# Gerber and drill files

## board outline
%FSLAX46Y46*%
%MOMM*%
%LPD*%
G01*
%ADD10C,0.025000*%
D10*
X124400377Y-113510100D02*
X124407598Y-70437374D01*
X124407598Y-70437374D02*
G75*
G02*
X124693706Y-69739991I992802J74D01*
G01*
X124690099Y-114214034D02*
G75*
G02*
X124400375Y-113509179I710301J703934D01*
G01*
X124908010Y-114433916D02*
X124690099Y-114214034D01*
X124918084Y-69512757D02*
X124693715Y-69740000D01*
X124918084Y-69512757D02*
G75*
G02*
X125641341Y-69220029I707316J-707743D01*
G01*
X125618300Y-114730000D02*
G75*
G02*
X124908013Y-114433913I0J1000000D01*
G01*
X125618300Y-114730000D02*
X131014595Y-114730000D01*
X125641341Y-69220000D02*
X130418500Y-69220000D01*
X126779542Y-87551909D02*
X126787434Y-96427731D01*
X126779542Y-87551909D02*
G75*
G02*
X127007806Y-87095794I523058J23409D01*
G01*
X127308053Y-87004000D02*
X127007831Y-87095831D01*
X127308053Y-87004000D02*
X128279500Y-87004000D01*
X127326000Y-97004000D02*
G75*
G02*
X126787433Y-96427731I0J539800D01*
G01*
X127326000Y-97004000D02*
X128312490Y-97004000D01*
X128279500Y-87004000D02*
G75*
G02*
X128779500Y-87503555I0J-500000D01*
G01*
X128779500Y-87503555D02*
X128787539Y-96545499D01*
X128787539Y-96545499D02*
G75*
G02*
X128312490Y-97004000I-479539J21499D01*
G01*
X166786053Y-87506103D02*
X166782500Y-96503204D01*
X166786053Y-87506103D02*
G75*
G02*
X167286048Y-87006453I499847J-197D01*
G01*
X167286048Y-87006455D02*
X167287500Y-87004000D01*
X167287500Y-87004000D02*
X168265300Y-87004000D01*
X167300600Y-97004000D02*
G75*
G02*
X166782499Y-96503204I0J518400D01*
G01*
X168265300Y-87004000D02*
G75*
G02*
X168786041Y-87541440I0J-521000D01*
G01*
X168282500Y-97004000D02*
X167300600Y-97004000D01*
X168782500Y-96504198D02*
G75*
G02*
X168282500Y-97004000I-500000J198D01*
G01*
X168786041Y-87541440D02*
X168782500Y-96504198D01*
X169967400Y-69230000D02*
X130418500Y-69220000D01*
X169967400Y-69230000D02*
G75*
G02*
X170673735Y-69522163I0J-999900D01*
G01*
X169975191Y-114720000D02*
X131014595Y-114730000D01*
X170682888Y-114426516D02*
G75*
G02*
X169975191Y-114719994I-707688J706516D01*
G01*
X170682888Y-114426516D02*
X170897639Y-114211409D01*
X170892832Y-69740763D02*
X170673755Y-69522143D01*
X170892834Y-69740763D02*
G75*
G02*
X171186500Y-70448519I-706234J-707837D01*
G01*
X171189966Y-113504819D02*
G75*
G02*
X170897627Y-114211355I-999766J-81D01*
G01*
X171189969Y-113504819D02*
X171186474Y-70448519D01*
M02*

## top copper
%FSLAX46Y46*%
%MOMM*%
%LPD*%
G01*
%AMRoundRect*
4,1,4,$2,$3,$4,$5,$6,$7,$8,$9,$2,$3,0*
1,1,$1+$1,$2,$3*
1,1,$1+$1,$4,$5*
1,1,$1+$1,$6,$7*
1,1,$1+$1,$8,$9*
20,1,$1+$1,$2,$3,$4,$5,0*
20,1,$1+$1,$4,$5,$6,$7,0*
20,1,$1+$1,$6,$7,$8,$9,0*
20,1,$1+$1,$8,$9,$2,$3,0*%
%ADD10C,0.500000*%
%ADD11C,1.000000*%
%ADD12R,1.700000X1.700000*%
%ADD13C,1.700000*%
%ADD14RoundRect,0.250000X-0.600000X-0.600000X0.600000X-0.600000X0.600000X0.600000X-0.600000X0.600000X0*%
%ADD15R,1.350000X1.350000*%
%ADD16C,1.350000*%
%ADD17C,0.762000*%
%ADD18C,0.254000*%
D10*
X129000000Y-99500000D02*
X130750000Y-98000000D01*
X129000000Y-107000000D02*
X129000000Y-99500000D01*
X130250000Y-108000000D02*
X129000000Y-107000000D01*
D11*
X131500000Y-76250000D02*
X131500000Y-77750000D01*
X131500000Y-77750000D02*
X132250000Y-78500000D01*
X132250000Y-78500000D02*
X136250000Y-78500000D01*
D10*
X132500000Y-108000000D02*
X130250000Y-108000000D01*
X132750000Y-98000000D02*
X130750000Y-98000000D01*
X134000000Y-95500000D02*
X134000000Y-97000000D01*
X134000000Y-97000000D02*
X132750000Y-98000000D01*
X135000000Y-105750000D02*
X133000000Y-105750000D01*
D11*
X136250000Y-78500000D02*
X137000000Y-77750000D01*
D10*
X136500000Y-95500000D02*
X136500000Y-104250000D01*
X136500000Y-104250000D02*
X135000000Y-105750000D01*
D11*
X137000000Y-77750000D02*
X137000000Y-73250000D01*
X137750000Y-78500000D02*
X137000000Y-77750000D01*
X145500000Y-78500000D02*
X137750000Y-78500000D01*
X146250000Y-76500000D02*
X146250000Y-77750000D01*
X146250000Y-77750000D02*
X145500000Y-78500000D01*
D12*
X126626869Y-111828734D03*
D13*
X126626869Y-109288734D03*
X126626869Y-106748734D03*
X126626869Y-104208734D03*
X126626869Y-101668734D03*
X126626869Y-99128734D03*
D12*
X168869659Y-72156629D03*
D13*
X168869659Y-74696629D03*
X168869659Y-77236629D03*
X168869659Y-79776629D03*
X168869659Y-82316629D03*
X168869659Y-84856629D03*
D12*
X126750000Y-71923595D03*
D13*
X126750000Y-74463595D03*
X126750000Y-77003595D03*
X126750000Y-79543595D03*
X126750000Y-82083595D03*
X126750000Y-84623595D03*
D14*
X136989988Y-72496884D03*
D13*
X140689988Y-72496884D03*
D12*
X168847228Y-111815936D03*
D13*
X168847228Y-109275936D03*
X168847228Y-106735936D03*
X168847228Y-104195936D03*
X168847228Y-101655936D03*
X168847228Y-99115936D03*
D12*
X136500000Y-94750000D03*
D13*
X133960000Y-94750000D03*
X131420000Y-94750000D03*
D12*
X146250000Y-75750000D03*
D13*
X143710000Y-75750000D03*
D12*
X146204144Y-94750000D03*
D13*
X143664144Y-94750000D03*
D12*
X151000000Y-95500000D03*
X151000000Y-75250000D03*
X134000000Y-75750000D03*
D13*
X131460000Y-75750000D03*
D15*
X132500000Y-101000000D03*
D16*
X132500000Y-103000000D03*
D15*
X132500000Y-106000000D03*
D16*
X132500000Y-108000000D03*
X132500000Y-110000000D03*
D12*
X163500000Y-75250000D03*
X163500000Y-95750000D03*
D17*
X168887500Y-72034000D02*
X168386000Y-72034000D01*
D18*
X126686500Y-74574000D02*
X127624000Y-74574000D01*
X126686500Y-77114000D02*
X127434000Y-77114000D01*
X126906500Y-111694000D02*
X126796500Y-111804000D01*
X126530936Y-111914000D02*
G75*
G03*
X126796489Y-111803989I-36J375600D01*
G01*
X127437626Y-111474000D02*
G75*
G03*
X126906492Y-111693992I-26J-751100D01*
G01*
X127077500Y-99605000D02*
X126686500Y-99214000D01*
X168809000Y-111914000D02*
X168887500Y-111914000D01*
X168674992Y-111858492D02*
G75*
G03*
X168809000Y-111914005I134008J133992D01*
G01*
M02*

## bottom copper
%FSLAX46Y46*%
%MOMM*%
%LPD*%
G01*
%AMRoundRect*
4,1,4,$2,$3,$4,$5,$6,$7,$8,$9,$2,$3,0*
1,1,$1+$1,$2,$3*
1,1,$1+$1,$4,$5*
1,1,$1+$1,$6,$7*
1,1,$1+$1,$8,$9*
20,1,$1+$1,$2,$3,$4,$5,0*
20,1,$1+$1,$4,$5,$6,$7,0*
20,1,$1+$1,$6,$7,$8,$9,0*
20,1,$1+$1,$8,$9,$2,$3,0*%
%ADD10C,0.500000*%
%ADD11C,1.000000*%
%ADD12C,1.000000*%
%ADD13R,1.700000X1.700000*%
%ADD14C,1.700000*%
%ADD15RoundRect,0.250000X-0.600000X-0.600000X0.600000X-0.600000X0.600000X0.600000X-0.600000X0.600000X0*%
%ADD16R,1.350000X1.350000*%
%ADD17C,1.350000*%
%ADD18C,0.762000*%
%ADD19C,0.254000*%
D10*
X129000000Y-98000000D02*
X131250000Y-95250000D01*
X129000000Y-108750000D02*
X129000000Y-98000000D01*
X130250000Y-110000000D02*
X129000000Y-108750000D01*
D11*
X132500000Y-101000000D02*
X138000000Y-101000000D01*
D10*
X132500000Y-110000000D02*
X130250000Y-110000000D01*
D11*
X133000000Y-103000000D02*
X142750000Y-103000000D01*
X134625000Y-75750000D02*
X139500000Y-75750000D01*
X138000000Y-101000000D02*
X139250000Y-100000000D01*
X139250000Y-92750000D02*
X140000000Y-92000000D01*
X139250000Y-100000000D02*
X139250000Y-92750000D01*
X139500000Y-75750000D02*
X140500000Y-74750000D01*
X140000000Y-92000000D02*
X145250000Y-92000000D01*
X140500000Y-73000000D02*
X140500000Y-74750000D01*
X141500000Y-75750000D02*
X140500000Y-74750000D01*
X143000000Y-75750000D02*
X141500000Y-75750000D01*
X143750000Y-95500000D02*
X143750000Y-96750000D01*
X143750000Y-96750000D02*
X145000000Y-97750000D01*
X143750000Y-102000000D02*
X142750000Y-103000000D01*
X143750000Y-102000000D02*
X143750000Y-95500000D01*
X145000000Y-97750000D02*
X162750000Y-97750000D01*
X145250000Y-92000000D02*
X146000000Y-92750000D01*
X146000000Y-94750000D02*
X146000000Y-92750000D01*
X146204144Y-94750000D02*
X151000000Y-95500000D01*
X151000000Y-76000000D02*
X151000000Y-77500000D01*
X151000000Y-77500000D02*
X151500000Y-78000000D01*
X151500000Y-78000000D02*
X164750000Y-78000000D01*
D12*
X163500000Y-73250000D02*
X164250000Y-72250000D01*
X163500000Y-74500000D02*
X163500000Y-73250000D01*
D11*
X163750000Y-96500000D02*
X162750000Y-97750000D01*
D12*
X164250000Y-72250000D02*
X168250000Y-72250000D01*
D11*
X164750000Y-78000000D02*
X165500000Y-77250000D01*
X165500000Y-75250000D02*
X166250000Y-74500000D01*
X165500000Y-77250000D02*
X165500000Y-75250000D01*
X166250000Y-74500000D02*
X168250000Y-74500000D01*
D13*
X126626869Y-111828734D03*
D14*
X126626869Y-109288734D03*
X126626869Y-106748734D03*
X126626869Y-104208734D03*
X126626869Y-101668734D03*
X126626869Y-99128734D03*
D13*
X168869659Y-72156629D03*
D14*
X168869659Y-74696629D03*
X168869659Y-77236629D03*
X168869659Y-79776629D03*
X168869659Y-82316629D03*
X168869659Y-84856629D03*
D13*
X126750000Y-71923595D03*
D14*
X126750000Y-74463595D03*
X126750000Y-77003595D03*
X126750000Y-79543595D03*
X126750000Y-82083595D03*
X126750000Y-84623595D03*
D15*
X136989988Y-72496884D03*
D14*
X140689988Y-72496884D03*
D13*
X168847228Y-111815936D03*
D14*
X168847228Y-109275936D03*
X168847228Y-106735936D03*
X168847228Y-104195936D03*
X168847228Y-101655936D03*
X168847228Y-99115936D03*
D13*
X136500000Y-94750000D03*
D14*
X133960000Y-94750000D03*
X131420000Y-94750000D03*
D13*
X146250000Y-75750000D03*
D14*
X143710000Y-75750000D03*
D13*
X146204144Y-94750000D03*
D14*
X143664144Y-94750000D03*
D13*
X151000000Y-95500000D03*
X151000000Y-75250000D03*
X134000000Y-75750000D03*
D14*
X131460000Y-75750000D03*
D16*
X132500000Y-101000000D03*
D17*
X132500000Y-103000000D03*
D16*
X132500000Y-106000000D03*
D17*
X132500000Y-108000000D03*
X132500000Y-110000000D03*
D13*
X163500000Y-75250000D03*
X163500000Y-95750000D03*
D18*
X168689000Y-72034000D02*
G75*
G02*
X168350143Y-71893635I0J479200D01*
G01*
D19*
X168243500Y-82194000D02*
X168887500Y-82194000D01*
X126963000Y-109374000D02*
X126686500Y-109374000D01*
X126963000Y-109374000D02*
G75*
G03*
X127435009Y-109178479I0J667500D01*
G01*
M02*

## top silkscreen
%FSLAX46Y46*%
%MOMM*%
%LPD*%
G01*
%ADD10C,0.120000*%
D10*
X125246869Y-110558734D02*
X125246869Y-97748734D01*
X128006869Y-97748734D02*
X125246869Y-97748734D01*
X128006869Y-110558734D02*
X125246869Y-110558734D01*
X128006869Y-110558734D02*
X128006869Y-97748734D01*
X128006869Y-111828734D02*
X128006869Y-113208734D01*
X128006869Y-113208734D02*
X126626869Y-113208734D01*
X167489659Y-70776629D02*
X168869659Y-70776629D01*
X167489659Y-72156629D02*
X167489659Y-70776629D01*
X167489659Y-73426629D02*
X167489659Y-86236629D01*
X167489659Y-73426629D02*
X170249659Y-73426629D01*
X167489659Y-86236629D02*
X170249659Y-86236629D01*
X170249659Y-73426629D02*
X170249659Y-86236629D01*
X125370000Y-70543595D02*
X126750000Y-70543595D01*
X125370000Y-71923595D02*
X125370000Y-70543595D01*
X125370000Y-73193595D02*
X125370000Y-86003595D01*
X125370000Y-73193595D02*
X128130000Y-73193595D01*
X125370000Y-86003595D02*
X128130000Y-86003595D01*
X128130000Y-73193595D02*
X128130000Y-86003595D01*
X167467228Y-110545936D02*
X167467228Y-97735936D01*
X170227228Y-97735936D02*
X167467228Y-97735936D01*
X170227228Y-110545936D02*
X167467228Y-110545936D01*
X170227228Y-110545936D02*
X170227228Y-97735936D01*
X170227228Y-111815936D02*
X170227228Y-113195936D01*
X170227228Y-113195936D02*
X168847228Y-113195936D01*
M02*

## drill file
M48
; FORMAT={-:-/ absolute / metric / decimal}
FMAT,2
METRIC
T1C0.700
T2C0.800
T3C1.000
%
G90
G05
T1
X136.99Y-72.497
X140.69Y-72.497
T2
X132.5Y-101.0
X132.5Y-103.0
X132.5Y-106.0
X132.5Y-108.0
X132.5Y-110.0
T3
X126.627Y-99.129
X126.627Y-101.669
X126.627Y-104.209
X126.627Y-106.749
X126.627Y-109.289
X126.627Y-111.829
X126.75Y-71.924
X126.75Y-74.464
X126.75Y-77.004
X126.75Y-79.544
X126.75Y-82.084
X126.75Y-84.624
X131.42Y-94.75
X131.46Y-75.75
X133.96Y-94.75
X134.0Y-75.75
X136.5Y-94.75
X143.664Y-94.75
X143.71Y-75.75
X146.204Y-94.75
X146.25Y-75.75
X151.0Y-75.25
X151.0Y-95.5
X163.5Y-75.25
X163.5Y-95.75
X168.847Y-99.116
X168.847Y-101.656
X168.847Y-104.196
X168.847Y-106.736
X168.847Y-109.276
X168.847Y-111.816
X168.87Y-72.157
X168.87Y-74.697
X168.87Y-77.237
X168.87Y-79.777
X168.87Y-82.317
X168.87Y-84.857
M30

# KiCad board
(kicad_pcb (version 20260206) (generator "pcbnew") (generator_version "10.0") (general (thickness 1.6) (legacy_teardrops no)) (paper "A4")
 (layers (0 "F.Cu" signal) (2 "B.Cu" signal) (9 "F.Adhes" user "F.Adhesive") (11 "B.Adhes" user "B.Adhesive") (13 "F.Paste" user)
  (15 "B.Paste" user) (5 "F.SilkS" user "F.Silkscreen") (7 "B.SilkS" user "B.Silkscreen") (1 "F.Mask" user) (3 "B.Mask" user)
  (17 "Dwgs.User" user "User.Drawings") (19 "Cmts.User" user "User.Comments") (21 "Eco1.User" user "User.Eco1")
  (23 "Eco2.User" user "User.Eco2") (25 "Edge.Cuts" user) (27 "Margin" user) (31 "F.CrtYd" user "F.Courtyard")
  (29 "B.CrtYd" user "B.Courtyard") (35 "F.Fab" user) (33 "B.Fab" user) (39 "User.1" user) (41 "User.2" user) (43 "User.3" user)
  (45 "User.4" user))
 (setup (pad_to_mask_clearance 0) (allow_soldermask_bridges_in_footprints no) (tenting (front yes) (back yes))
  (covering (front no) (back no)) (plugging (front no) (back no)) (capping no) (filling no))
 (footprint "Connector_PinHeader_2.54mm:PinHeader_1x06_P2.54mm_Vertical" (layer "F.Cu") (at 126.626869 111.828734 180)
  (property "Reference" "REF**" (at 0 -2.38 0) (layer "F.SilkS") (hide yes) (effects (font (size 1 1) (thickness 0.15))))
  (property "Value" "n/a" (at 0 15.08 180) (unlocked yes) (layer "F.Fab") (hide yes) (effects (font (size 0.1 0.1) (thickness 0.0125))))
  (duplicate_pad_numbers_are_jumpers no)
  (fp_line (start 1.38 1.27) (end 1.38 14.08) (stroke (width 0.12) (type solid)) (layer "F.SilkS"))
  (fp_line (start -1.38 14.08) (end 1.38 14.08) (stroke (width 0.12) (type solid)) (layer "F.SilkS"))
  (fp_line (start -1.38 1.27) (end 1.38 1.27) (stroke (width 0.12) (type solid)) (layer "F.SilkS"))
  (fp_line (start -1.38 1.27) (end -1.38 14.08) (stroke (width 0.12) (type solid)) (layer "F.SilkS"))
  (fp_line (start -1.38 0) (end -1.38 -1.38) (stroke (width 0.12) (type solid)) (layer "F.SilkS"))
  (fp_line (start -1.38 -1.38) (end 0 -1.38) (stroke (width 0.12) (type solid)) (layer "F.SilkS"))
  (pad "1" thru_hole rect (at 0 0 180) (size 1.7 1.7) (drill 1) (layers "*.Cu" "*.Mask") (remove_unused_layers no))
  (pad "2" thru_hole circle (at 0 2.54 180) (size 1.7 1.7) (drill 1) (layers "*.Cu" "*.Mask") (remove_unused_layers no))
  (pad "3" thru_hole circle (at 0 5.08 180) (size 1.7 1.7) (drill 1) (layers "*.Cu" "*.Mask") (remove_unused_layers no))
  (pad "4" thru_hole circle (at 0 7.62 180) (size 1.7 1.7) (drill 1) (layers "*.Cu" "*.Mask") (remove_unused_layers no))
  (pad "5" thru_hole circle (at 0 10.16 180) (size 1.7 1.7) (drill 1) (layers "*.Cu" "*.Mask") (remove_unused_layers no))
  (pad "6" thru_hole circle (at 0 12.7 180) (size 1.7 1.7) (drill 1) (layers "*.Cu" "*.Mask") (remove_unused_layers no)))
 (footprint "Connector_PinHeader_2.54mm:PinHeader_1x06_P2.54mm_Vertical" (layer "F.Cu") (at 168.869659 72.156629)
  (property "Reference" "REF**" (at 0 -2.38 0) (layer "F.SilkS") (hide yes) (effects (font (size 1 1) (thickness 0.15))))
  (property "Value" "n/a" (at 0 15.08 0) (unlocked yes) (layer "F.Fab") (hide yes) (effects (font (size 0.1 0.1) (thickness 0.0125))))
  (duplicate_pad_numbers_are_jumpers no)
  (fp_line (start -1.38 -1.38) (end 0 -1.38) (stroke (width 0.12) (type solid)) (layer "F.SilkS"))
  (fp_line (start -1.38 0) (end -1.38 -1.38) (stroke (width 0.12) (type solid)) (layer "F.SilkS"))
  (fp_line (start -1.38 1.27) (end -1.38 14.08) (stroke (width 0.12) (type solid)) (layer "F.SilkS"))
  (fp_line (start -1.38 1.27) (end 1.38 1.27) (stroke (width 0.12) (type solid)) (layer "F.SilkS"))
  (fp_line (start -1.38 14.08) (end 1.38 14.08) (stroke (width 0.12) (type solid)) (layer "F.SilkS"))
  (fp_line (start 1.38 1.27) (end 1.38 14.08) (stroke (width 0.12) (type solid)) (layer "F.SilkS"))
  (pad "1" thru_hole rect (at 0 0) (size 1.7 1.7) (drill 1) (layers "*.Cu" "*.Mask") (remove_unused_layers no))
  (pad "2" thru_hole circle (at 0 2.54) (size 1.7 1.7) (drill 1) (layers "*.Cu" "*.Mask") (remove_unused_layers no))
  (pad "3" thru_hole circle (at 0 5.08) (size 1.7 1.7) (drill 1) (layers "*.Cu" "*.Mask") (remove_unused_layers no))
  (pad "4" thru_hole circle (at 0 7.62) (size 1.7 1.7) (drill 1) (layers "*.Cu" "*.Mask") (remove_unused_layers no))
  (pad "5" thru_hole circle (at 0 10.16) (size 1.7 1.7) (drill 1) (layers "*.Cu" "*.Mask") (remove_unused_layers no))
  (pad "6" thru_hole circle (at 0 12.7) (size 1.7 1.7) (drill 1) (layers "*.Cu" "*.Mask") (remove_unused_layers no)))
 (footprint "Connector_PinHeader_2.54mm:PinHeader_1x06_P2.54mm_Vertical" (layer "F.Cu") (at 126.75 71.923595)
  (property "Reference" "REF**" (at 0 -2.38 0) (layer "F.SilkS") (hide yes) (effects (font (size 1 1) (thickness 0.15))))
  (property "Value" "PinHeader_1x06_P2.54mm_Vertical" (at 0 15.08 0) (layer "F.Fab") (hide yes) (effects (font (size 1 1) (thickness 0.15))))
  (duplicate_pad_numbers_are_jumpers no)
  (fp_line (start -1.38 -1.38) (end 0 -1.38) (stroke (width 0.12) (type solid)) (layer "F.SilkS"))
  (fp_line (start -1.38 0) (end -1.38 -1.38) (stroke (width 0.12) (type solid)) (layer "F.SilkS"))
  (fp_line (start -1.38 1.27) (end -1.38 14.08) (stroke (width 0.12) (type solid)) (layer "F.SilkS"))
  (fp_line (start -1.38 1.27) (end 1.38 1.27) (stroke (width 0.12) (type solid)) (layer "F.SilkS"))
  (fp_line (start -1.38 14.08) (end 1.38 14.08) (stroke (width 0.12) (type solid)) (layer "F.SilkS"))
  (fp_line (start 1.38 1.27) (end 1.38 14.08) (stroke (width 0.12) (type solid)) (layer "F.SilkS"))
  (pad "1" thru_hole rect (at 0 0) (size 1.7 1.7) (drill 1) (layers "*.Cu" "*.Mask") (remove_unused_layers no))
  (pad "2" thru_hole circle (at 0 2.54) (size 1.7 1.7) (drill 1) (layers "*.Cu" "*.Mask") (remove_unused_layers no))
  (pad "3" thru_hole circle (at 0 5.08) (size 1.7 1.7) (drill 1) (layers "*.Cu" "*.Mask") (remove_unused_layers no))
  (pad "4" thru_hole circle (at 0 7.62) (size 1.7 1.7) (drill 1) (layers "*.Cu" "*.Mask") (remove_unused_layers no))
  (pad "5" thru_hole circle (at 0 10.16) (size 1.7 1.7) (drill 1) (layers "*.Cu" "*.Mask") (remove_unused_layers no))
  (pad "6" thru_hole circle (at 0 12.7) (size 1.7 1.7) (drill 1) (layers "*.Cu" "*.Mask") (remove_unused_layers no)))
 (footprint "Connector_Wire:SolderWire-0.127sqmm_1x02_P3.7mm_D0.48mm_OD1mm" (layer "F.Cu") (at 136.989988 72.496884)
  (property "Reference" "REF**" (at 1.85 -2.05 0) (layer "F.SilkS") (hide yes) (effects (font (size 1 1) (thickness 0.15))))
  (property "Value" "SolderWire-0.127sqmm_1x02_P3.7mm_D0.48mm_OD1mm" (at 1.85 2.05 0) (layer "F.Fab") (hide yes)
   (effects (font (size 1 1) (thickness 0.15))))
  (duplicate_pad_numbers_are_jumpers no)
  (pad "1" thru_hole roundrect (at 0 0) (size 1.7 1.7) (drill 0.7) (layers "*.Cu" "*.Mask") (remove_unused_layers no)
   (roundrect_rratio 0.147059))
  (pad "2" thru_hole circle (at 3.7 0) (size 1.7 1.7) (drill 0.7) (layers "*.Cu" "*.Mask") (remove_unused_layers no)))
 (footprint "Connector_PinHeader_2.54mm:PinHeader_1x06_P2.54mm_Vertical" (layer "F.Cu") (at 168.847228 111.815936 180)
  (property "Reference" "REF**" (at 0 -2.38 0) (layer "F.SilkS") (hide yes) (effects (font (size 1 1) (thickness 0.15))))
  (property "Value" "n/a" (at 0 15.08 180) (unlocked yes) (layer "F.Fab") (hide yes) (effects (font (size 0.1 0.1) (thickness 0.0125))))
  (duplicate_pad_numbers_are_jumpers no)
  (fp_line (start 1.38 1.27) (end 1.38 14.08) (stroke (width 0.12) (type solid)) (layer "F.SilkS"))
  (fp_line (start -1.38 14.08) (end 1.38 14.08) (stroke (width 0.12) (type solid)) (layer "F.SilkS"))
  (fp_line (start -1.38 1.27) (end 1.38 1.27) (stroke (width 0.12) (type solid)) (layer "F.SilkS"))
  (fp_line (start -1.38 1.27) (end -1.38 14.08) (stroke (width 0.12) (type solid)) (layer "F.SilkS"))
  (fp_line (start -1.38 0) (end -1.38 -1.38) (stroke (width 0.12) (type solid)) (layer "F.SilkS"))
  (fp_line (start -1.38 -1.38) (end 0 -1.38) (stroke (width 0.12) (type solid)) (layer "F.SilkS"))
  (pad "1" thru_hole rect (at 0 0 180) (size 1.7 1.7) (drill 1) (layers "*.Cu" "*.Mask") (remove_unused_layers no))
  (pad "2" thru_hole circle (at 0 2.54 180) (size 1.7 1.7) (drill 1) (layers "*.Cu" "*.Mask") (remove_unused_layers no))
  (pad "3" thru_hole circle (at 0 5.08 180) (size 1.7 1.7) (drill 1) (layers "*.Cu" "*.Mask") (remove_unused_layers no))
  (pad "4" thru_hole circle (at 0 7.62 180) (size 1.7 1.7) (drill 1) (layers "*.Cu" "*.Mask") (remove_unused_layers no))
  (pad "5" thru_hole circle (at 0 10.16 180) (size 1.7 1.7) (drill 1) (layers "*.Cu" "*.Mask") (remove_unused_layers no))
  (pad "6" thru_hole circle (at 0 12.7 180) (size 1.7 1.7) (drill 1) (layers "*.Cu" "*.Mask") (remove_unused_layers no)))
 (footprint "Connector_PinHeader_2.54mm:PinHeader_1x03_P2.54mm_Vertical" (layer "B.Cu") (at 136.5 94.75 90)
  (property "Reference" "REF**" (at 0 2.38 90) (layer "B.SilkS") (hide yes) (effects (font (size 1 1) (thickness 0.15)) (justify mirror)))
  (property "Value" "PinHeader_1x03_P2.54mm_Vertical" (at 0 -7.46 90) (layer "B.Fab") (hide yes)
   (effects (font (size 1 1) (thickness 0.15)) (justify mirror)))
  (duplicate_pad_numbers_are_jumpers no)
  (pad "1" thru_hole rect (at 0 0 90) (size 1.7 1.7) (drill 1) (layers "*.Cu" "*.Mask") (remove_unused_layers no))
  (pad "2" thru_hole circle (at 0 -2.54 90) (size 1.7 1.7) (drill 1) (layers "*.Cu" "*.Mask") (remove_unused_layers no))
  (pad "3" thru_hole circle (at 0 -5.08 90) (size 1.7 1.7) (drill 1) (layers "*.Cu" "*.Mask") (remove_unused_layers no)))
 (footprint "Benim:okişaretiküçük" (layer "B.Cu") (at 149 71.5 135)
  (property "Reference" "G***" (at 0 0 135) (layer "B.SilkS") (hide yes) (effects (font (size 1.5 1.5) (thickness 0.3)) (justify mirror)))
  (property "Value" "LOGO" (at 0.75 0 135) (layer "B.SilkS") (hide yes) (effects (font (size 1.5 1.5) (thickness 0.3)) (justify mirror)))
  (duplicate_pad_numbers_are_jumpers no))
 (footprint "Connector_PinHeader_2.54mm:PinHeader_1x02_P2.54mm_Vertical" (layer "B.Cu") (at 146.25 75.75 90)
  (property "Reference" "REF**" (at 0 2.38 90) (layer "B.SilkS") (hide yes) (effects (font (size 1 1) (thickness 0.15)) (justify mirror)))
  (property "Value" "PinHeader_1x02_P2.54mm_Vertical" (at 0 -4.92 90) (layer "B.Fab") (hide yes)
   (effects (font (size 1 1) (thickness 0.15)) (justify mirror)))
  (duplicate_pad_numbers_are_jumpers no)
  (pad "1" thru_hole rect (at 0 0 90) (size 1.7 1.7) (drill 1) (layers "*.Cu" "*.Mask") (remove_unused_layers no))
  (pad "2" thru_hole circle (at 0 -2.54 90) (size 1.7 1.7) (drill 1) (layers "*.Cu" "*.Mask") (remove_unused_layers no)))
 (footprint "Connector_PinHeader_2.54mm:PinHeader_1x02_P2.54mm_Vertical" (layer "B.Cu") (at 146.204144 94.75 90)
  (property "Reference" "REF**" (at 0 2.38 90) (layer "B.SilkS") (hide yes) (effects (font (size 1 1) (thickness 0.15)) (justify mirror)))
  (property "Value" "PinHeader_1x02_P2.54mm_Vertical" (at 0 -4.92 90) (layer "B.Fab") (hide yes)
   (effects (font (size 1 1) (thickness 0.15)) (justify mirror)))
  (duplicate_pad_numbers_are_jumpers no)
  (pad "1" thru_hole rect (at 0 0 90) (size 1.7 1.7) (drill 1) (layers "*.Cu" "*.Mask") (remove_unused_layers no))
  (pad "2" thru_hole circle (at 0 -2.54 90) (size 1.7 1.7) (drill 1) (layers "*.Cu" "*.Mask") (remove_unused_layers no)))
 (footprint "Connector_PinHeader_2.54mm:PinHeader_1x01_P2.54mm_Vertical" (layer "B.Cu") (at 151 95.5 180)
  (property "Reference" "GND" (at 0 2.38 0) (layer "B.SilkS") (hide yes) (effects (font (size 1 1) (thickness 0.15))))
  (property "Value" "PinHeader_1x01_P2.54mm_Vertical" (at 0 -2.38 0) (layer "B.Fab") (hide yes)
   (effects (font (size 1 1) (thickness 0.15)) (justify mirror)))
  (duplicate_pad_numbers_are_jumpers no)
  (pad "1" thru_hole rect (at 0 0 180) (size 1.7 1.7) (drill 1) (layers "*.Cu" "*.Mask") (remove_unused_layers no)))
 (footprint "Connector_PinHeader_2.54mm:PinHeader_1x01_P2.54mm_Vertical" (layer "B.Cu") (at 151 75.25 180)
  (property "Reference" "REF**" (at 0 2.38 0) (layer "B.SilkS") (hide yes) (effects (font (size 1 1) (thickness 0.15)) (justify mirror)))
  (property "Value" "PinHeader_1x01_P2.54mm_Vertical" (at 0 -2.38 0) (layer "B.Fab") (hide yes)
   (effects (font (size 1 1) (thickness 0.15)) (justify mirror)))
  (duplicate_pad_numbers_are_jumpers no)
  (pad "1" thru_hole rect (at 0 0 180) (size 1.7 1.7) (drill 1) (layers "*.Cu" "*.Mask") (remove_unused_layers no)))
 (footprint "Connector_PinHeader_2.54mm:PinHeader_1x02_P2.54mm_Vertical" (layer "B.Cu") (at 134 75.75 90)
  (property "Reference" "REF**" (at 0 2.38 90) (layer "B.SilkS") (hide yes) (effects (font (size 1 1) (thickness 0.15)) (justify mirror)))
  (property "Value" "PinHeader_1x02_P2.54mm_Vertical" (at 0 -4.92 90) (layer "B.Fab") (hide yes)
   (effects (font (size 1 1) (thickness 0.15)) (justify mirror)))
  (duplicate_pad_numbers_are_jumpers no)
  (pad "1" thru_hole rect (at 0 0 90) (size 1.7 1.7) (drill 1) (layers "*.Cu" "*.Mask") (remove_unused_layers no))
  (pad "2" thru_hole circle (at 0 -2.54 90) (size 1.7 1.7) (drill 1) (layers "*.Cu" "*.Mask") (remove_unused_layers no)))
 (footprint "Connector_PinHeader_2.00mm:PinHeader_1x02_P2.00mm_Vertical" (layer "B.Cu") (at 132.5 101 180)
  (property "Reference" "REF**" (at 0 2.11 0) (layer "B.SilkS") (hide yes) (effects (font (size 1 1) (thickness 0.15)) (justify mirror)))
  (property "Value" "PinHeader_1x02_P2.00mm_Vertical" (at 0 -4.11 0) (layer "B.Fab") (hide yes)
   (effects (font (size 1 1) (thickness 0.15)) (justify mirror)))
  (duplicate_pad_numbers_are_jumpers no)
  (pad "1" thru_hole rect (at 0 0 180) (size 1.35 1.35) (drill 0.8) (layers "*.Cu" "*.Mask") (remove_unused_layers no))
  (pad "2" thru_hole circle (at 0 -2 180) (size 1.35 1.35) (drill 0.8) (layers "*.Cu" "*.Mask") (remove_unused_layers no)))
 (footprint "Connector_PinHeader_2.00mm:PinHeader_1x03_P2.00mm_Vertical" (layer "B.Cu") (at 132.5 106 180)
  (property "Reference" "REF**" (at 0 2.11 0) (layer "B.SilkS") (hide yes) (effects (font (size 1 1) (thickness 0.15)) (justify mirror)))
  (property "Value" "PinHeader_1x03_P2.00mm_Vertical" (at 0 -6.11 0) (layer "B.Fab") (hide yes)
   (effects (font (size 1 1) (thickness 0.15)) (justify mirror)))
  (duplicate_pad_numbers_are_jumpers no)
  (pad "1" thru_hole rect (at 0 0 180) (size 1.35 1.35) (drill 0.8) (layers "*.Cu" "*.Mask") (remove_unused_layers no))
  (pad "2" thru_hole circle (at 0 -2 180) (size 1.35 1.35) (drill 0.8) (layers "*.Cu" "*.Mask") (remove_unused_layers no))
  (pad "3" thru_hole circle (at 0 -4 180) (size 1.35 1.35) (drill 0.8) (layers "*.Cu" "*.Mask") (remove_unused_layers no)))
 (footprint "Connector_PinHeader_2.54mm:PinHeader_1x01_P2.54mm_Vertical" (layer "B.Cu") (at 163.5 75.25 180)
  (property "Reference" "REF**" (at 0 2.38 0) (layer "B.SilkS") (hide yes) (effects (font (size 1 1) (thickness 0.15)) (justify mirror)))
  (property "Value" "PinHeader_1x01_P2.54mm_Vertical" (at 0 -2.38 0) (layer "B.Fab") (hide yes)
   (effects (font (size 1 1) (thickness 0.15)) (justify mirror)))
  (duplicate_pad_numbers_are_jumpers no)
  (pad "1" thru_hole rect (at 0 0 180) (size 1.7 1.7) (drill 1) (layers "*.Cu" "*.Mask") (remove_unused_layers no)))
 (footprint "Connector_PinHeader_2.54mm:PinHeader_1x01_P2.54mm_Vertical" (layer "B.Cu") (at 163.5 95.75 180)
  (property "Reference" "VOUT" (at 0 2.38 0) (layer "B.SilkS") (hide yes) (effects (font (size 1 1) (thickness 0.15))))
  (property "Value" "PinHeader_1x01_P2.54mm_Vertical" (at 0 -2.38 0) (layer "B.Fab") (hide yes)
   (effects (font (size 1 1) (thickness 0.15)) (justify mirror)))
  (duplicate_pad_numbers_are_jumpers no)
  (pad "1" thru_hole rect (at 0 0 180) (size 1.7 1.7) (drill 1) (layers "*.Cu" "*.Mask") (remove_unused_layers no)))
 (gr_line (start 129 99.5) (end 130.75 98) (stroke (width 0.5) (type solid)) (layer "F.Cu"))
 (gr_line (start 129 107) (end 129 99.5) (stroke (width 0.5) (type solid)) (layer "F.Cu"))
 (gr_line (start 130.25 108) (end 129 107) (stroke (width 0.5) (type solid)) (layer "F.Cu"))
 (gr_line (start 131.5 76.25) (end 131.5 77.75) (stroke (width 1) (type solid)) (layer "F.Cu"))
 (gr_line (start 131.5 77.75) (end 132.25 78.5) (stroke (width 1) (type solid)) (layer "F.Cu"))
 (gr_line (start 132.25 78.5) (end 136.25 78.5) (stroke (width 1) (type solid)) (layer "F.Cu"))
 (gr_line (start 132.5 108) (end 130.25 108) (stroke (width 0.5) (type solid)) (layer "F.Cu"))
 (gr_line (start 132.75 98) (end 130.75 98) (stroke (width 0.5) (type solid)) (layer "F.Cu"))
 (gr_line (start 134 95.5) (end 134 97) (stroke (width 0.5) (type solid)) (layer "F.Cu"))
 (gr_line (start 134 97) (end 132.75 98) (stroke (width 0.5) (type solid)) (layer "F.Cu"))
 (gr_line (start 135 105.75) (end 133 105.75) (stroke (width 0.5) (type solid)) (layer "F.Cu"))
 (gr_line (start 136.25 78.5) (end 137 77.75) (stroke (width 1) (type solid)) (layer "F.Cu"))
 (gr_line (start 136.5 95.5) (end 136.5 104.25) (stroke (width 0.5) (type solid)) (layer "F.Cu"))
 (gr_line (start 136.5 104.25) (end 135 105.75) (stroke (width 0.5) (type solid)) (layer "F.Cu"))
 (gr_line (start 137 77.75) (end 137 73.25) (stroke (width 1) (type solid)) (layer "F.Cu"))
 (gr_line (start 137.75 78.5) (end 137 77.75) (stroke (width 1) (type solid)) (layer "F.Cu"))
 (gr_line (start 145.5 78.5) (end 137.75 78.5) (stroke (width 1) (type solid)) (layer "F.Cu"))
 (gr_line (start 146.25 76.5) (end 146.25 77.75) (stroke (width 1) (type solid)) (layer "F.Cu"))
 (gr_line (start 146.25 77.75) (end 145.5 78.5) (stroke (width 1) (type solid)) (layer "F.Cu"))
 (gr_line (start 129 98) (end 131.25 95.25) (stroke (width 0.5) (type solid)) (layer "B.Cu"))
 (gr_line (start 129 108.75) (end 129 98) (stroke (width 0.5) (type solid)) (layer "B.Cu"))
 (gr_line (start 130.25 110) (end 129 108.75) (stroke (width 0.5) (type solid)) (layer "B.Cu"))
 (gr_line (start 132.5 101) (end 138 101) (stroke (width 1) (type solid)) (layer "B.Cu"))
 (gr_line (start 132.5 110) (end 130.25 110) (stroke (width 0.5) (type solid)) (layer "B.Cu"))
 (gr_line (start 133 103) (end 142.75 103) (stroke (width 1) (type solid)) (layer "B.Cu"))
 (gr_line (start 134.625 75.75) (end 139.5 75.75) (stroke (width 1) (type solid)) (layer "B.Cu"))
 (gr_line (start 138 101) (end 139.25 100) (stroke (width 1) (type solid)) (layer "B.Cu"))
 (gr_line (start 139.25 92.75) (end 140 92) (stroke (width 1) (type solid)) (layer "B.Cu"))
 (gr_line (start 139.25 100) (end 139.25 92.75) (stroke (width 1) (type solid)) (layer "B.Cu"))
 (gr_line (start 139.5 75.75) (end 140.5 74.75) (stroke (width 1) (type solid)) (layer "B.Cu"))
 (gr_line (start 140 92) (end 145.25 92) (stroke (width 1) (type solid)) (layer "B.Cu"))
 (gr_line (start 140.5 73) (end 140.5 74.75) (stroke (width 1) (type solid)) (layer "B.Cu"))
 (gr_line (start 141.5 75.75) (end 140.5 74.75) (stroke (width 1) (type solid)) (layer "B.Cu"))
 (gr_line (start 143 75.75) (end 141.5 75.75) (stroke (width 1) (type solid)) (layer "B.Cu"))
 (gr_line (start 143.75 95.5) (end 143.75 96.75) (stroke (width 1) (type solid)) (layer "B.Cu"))
 (gr_line (start 143.75 96.75) (end 145 97.75) (stroke (width 1) (type solid)) (layer "B.Cu"))
 (gr_line (start 143.75 102) (end 142.75 103) (stroke (width 1) (type solid)) (layer "B.Cu"))
 (gr_line (start 143.75 102) (end 143.75 95.5) (stroke (width 1) (type solid)) (layer "B.Cu"))
 (gr_line (start 145 97.75) (end 162.75 97.75) (stroke (width 1) (type solid)) (layer "B.Cu"))
 (gr_line (start 145.25 92) (end 146 92.75) (stroke (width 1) (type solid)) (layer "B.Cu"))
 (gr_line (start 146 94.75) (end 146 92.75) (stroke (width 1) (type solid)) (layer "B.Cu"))
 (gr_line (start 146.204144 94.75) (end 151 95.5) (stroke (width 1) (type solid)) (layer "B.Cu"))
 (gr_line (start 151 76) (end 151 77.5) (stroke (width 1) (type solid)) (layer "B.Cu"))
 (gr_line (start 151 77.5) (end 151.5 78) (stroke (width 1) (type solid)) (layer "B.Cu"))
 (gr_line (start 151.5 78) (end 164.75 78) (stroke (width 1) (type solid)) (layer "B.Cu"))
 (gr_line (start 163.5 73.25) (end 164.25 72.25) (stroke (width 1) (type solid)) (layer "B.Cu") (net "VBUS"))
 (gr_line (start 163.5 74.5) (end 163.5 73.25) (stroke (width 1) (type solid)) (layer "B.Cu") (net "VBUS"))
 (gr_line (start 163.75 96.5) (end 162.75 97.75) (stroke (width 1) (type solid)) (layer "B.Cu"))
 (gr_line (start 164.25 72.25) (end 168.25 72.25) (stroke (width 1) (type solid)) (layer "B.Cu") (net "VBUS"))
 (gr_line (start 164.75 78) (end 165.5 77.25) (stroke (width 1) (type solid)) (layer "B.Cu"))
 (gr_line (start 165.5 75.25) (end 166.25 74.5) (stroke (width 1) (type solid)) (layer "B.Cu"))
 (gr_line (start 165.5 77.25) (end 165.5 75.25) (stroke (width 1) (type solid)) (layer "B.Cu"))
 (gr_line (start 166.25 74.5) (end 168.25 74.5) (stroke (width 1) (type solid)) (layer "B.Cu"))
 (gr_line (start 124.400377 113.5101) (end 124.407598 70.437374) (stroke (width 0.025) (type solid)) (layer "Edge.Cuts"))
 (gr_arc (start 124.407598 70.437374) (mid 124.481894 70.060475) (end 124.693715 69.74) (stroke (width 0.025) (type default))
  (layer "Edge.Cuts"))
 (gr_arc (start 124.690099 114.214034) (mid 124.475465 113.890292) (end 124.400377 113.509179) (stroke (width 0.025) (type default))
  (layer "Edge.Cuts"))
 (gr_line (start 124.90801 114.433916) (end 124.690099 114.214034) (stroke (width 0.025) (type solid)) (layer "Edge.Cuts"))
 (gr_line (start 124.918084 69.512757) (end 124.693715 69.74) (stroke (width 0.025) (type solid)) (layer "Edge.Cuts"))
 (gr_arc (start 124.918084 69.512757) (mid 125.242506 69.296048) (end 125.641341 69.22) (stroke (width 0.025) (type default))
  (layer "Edge.Cuts"))
 (gr_arc (start 125.6183 114.73) (mid 125.233531 114.653016) (end 124.90801 114.433916) (stroke (width 0.025) (type default))
  (layer "Edge.Cuts"))
 (gr_line (start 125.6183 114.73) (end 131.014595 114.73) (stroke (width 0.025) (type solid)) (layer "Edge.Cuts"))
 (gr_line (start 125.641341 69.22) (end 130.4185 69.22) (stroke (width 0.025) (type solid)) (layer "Edge.Cuts"))
 (gr_line (start 126.779542 87.551909) (end 126.787434 96.427731) (stroke (width 0.025) (type default)) (layer "Edge.Cuts"))
 (gr_arc (start 126.779542 87.551909) (mid 126.940006 87.150841) (end 127.007831 87.095831) (stroke (width 0.025) (type default))
  (layer "Edge.Cuts"))
 (gr_line (start 127.308053 87.004) (end 127.007831 87.095831) (stroke (width 0.025) (type default)) (layer "Edge.Cuts"))
 (gr_line (start 127.308053 87.004) (end 128.2795 87.004) (stroke (width 0.025) (type default)) (layer "Edge.Cuts"))
 (gr_arc (start 127.326 97.004) (mid 126.958691 96.859782) (end 126.787434 96.427731) (stroke (width 0.025) (type default))
  (layer "Edge.Cuts"))
 (gr_line (start 127.326 97.004) (end 128.31249 97.004) (stroke (width 0.025) (type solid)) (layer "Edge.Cuts"))
 (gr_arc (start 128.2795 87.004) (mid 128.633053 87.150447) (end 128.7795 87.503555) (stroke (width 0.025) (type default))
  (layer "Edge.Cuts"))
 (gr_line (start 128.7795 87.503555) (end 128.787539 96.545499) (stroke (width 0.025) (type default)) (layer "Edge.Cuts"))
 (gr_arc (start 128.787539 96.545499) (mid 128.655295 96.855375) (end 128.31249 97.004) (stroke (width 0.025) (type default))
  (layer "Edge.Cuts"))
 (gr_line (start 166.786053 87.506103) (end 166.7825 96.503204) (stroke (width 0.025) (type default)) (layer "Edge.Cuts"))
 (gr_arc (start 166.786053 87.506103) (mid 166.932457 87.152853) (end 167.286048 87.006455) (stroke (width 0.025) (type default))
  (layer "Edge.Cuts"))
 (gr_line (start 167.286048 87.006455) (end 167.2875 87.004) (stroke (width 0.025) (type default)) (layer "Edge.Cuts"))
 (gr_line (start 167.2875 87.004) (end 168.2653 87.004) (stroke (width 0.025) (type default)) (layer "Edge.Cuts"))
 (gr_arc (start 167.3006 97.004) (mid 166.941479 96.859467) (end 166.7825 96.503204) (stroke (width 0.025) (type default))
  (layer "Edge.Cuts"))
 (gr_arc (start 168.2653 87.004) (mid 168.627679 87.150667) (end 168.786041 87.54144) (stroke (width 0.025) (type default))
  (layer "Edge.Cuts"))
 (gr_line (start 168.2825 97.004) (end 167.3006 97.004) (stroke (width 0.025) (type default)) (layer "Edge.Cuts"))
 (gr_arc (start 168.7825 96.504198) (mid 168.636053 96.857553) (end 168.2825 97.004) (stroke (width 0.025) (type default))
  (layer "Edge.Cuts"))
 (gr_line (start 168.786041 87.54144) (end 168.7825 96.504198) (stroke (width 0.025) (type default)) (layer "Edge.Cuts"))
 (gr_line (start 169.9674 69.23) (end 130.4185 69.22) (stroke (width 0.025) (type solid)) (layer "Edge.Cuts"))
 (gr_arc (start 169.9674 69.23) (mid 170.349644 69.305928) (end 170.673755 69.522143) (stroke (width 0.025) (type default))
  (layer "Edge.Cuts"))
 (gr_line (start 169.975191 114.72) (end 131.014595 114.73) (stroke (width 0.025) (type solid)) (layer "Edge.Cuts"))
 (gr_arc (start 170.682888 114.426516) (mid 170.358258 114.643717) (end 169.975191 114.72) (stroke (width 0.025) (type solid))
  (layer "Edge.Cuts"))
 (gr_line (start 170.682888 114.426516) (end 170.897639 114.211409) (stroke (width 0.025) (type solid)) (layer "Edge.Cuts"))
 (gr_line (start 170.892832 69.740763) (end 170.673755 69.522143) (stroke (width 0.025) (type solid)) (layer "Edge.Cuts"))
 (gr_arc (start 170.892834 69.740763) (mid 171.110147 70.065419) (end 171.18647 70.448519) (stroke (width 0.025) (type default))
  (layer "Edge.Cuts"))
 (gr_arc (start 171.189966 113.504819) (mid 171.11402 113.887129) (end 170.897639 114.211367) (stroke (width 0.025) (type default))
  (layer "Edge.Cuts"))
 (gr_line (start 171.189969 113.504819) (end 171.186474 70.448519) (stroke (width 0.025) (type solid)) (layer "Edge.Cuts"))
 (segment (start 168.8875 72.034) (end 168.386 72.034) (width 0.762) (layer "F.Cu") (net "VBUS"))
 (arc (start 168.689 72.034) (mid 168.505609 71.997521) (end 168.350139 71.893639) (width 0.762) (layer "B.Cu") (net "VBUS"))
 (segment (start 126.6865 74.574) (end 127.624 74.574) (width 0.254) (layer "F.Cu") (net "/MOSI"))
 (segment (start 168.2435 82.194) (end 168.8875 82.194) (width 0.254) (layer "B.Cu") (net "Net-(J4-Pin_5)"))
 (segment (start 126.6865 77.114) (end 127.434 77.114) (width 0.254) (layer "F.Cu") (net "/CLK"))
 (segment (start 126.9065 111.694) (end 126.7965 111.804) (width 0.254) (layer "F.Cu") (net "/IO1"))
 (arc (start 126.530936 111.914) (mid 126.674658 111.885411) (end 126.7965 111.804) (width 0.254) (layer "F.Cu") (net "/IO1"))
 (arc (start 127.437626 111.474) (mid 127.150182 111.531176) (end 126.9065 111.694) (width 0.254) (layer "F.Cu") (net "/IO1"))
 (segment (start 127.0775 99.605) (end 126.6865 99.214) (width 0.254) (layer "F.Cu") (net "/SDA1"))
 (segment (start 168.809 111.914) (end 168.8875 111.914) (width 0.254) (layer "F.Cu") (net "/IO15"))
 (arc (start 168.674992 111.858492) (mid 168.736475 111.899573) (end 168.809 111.914) (width 0.254) (layer "F.Cu") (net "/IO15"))
 (segment (start 126.963 109.374) (end 126.6865 109.374) (width 0.254) (layer "B.Cu") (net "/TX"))
 (arc (start 126.963 109.374) (mid 127.218452 109.323187) (end 127.435014 109.178484) (width 0.254) (layer "B.Cu") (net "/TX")))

